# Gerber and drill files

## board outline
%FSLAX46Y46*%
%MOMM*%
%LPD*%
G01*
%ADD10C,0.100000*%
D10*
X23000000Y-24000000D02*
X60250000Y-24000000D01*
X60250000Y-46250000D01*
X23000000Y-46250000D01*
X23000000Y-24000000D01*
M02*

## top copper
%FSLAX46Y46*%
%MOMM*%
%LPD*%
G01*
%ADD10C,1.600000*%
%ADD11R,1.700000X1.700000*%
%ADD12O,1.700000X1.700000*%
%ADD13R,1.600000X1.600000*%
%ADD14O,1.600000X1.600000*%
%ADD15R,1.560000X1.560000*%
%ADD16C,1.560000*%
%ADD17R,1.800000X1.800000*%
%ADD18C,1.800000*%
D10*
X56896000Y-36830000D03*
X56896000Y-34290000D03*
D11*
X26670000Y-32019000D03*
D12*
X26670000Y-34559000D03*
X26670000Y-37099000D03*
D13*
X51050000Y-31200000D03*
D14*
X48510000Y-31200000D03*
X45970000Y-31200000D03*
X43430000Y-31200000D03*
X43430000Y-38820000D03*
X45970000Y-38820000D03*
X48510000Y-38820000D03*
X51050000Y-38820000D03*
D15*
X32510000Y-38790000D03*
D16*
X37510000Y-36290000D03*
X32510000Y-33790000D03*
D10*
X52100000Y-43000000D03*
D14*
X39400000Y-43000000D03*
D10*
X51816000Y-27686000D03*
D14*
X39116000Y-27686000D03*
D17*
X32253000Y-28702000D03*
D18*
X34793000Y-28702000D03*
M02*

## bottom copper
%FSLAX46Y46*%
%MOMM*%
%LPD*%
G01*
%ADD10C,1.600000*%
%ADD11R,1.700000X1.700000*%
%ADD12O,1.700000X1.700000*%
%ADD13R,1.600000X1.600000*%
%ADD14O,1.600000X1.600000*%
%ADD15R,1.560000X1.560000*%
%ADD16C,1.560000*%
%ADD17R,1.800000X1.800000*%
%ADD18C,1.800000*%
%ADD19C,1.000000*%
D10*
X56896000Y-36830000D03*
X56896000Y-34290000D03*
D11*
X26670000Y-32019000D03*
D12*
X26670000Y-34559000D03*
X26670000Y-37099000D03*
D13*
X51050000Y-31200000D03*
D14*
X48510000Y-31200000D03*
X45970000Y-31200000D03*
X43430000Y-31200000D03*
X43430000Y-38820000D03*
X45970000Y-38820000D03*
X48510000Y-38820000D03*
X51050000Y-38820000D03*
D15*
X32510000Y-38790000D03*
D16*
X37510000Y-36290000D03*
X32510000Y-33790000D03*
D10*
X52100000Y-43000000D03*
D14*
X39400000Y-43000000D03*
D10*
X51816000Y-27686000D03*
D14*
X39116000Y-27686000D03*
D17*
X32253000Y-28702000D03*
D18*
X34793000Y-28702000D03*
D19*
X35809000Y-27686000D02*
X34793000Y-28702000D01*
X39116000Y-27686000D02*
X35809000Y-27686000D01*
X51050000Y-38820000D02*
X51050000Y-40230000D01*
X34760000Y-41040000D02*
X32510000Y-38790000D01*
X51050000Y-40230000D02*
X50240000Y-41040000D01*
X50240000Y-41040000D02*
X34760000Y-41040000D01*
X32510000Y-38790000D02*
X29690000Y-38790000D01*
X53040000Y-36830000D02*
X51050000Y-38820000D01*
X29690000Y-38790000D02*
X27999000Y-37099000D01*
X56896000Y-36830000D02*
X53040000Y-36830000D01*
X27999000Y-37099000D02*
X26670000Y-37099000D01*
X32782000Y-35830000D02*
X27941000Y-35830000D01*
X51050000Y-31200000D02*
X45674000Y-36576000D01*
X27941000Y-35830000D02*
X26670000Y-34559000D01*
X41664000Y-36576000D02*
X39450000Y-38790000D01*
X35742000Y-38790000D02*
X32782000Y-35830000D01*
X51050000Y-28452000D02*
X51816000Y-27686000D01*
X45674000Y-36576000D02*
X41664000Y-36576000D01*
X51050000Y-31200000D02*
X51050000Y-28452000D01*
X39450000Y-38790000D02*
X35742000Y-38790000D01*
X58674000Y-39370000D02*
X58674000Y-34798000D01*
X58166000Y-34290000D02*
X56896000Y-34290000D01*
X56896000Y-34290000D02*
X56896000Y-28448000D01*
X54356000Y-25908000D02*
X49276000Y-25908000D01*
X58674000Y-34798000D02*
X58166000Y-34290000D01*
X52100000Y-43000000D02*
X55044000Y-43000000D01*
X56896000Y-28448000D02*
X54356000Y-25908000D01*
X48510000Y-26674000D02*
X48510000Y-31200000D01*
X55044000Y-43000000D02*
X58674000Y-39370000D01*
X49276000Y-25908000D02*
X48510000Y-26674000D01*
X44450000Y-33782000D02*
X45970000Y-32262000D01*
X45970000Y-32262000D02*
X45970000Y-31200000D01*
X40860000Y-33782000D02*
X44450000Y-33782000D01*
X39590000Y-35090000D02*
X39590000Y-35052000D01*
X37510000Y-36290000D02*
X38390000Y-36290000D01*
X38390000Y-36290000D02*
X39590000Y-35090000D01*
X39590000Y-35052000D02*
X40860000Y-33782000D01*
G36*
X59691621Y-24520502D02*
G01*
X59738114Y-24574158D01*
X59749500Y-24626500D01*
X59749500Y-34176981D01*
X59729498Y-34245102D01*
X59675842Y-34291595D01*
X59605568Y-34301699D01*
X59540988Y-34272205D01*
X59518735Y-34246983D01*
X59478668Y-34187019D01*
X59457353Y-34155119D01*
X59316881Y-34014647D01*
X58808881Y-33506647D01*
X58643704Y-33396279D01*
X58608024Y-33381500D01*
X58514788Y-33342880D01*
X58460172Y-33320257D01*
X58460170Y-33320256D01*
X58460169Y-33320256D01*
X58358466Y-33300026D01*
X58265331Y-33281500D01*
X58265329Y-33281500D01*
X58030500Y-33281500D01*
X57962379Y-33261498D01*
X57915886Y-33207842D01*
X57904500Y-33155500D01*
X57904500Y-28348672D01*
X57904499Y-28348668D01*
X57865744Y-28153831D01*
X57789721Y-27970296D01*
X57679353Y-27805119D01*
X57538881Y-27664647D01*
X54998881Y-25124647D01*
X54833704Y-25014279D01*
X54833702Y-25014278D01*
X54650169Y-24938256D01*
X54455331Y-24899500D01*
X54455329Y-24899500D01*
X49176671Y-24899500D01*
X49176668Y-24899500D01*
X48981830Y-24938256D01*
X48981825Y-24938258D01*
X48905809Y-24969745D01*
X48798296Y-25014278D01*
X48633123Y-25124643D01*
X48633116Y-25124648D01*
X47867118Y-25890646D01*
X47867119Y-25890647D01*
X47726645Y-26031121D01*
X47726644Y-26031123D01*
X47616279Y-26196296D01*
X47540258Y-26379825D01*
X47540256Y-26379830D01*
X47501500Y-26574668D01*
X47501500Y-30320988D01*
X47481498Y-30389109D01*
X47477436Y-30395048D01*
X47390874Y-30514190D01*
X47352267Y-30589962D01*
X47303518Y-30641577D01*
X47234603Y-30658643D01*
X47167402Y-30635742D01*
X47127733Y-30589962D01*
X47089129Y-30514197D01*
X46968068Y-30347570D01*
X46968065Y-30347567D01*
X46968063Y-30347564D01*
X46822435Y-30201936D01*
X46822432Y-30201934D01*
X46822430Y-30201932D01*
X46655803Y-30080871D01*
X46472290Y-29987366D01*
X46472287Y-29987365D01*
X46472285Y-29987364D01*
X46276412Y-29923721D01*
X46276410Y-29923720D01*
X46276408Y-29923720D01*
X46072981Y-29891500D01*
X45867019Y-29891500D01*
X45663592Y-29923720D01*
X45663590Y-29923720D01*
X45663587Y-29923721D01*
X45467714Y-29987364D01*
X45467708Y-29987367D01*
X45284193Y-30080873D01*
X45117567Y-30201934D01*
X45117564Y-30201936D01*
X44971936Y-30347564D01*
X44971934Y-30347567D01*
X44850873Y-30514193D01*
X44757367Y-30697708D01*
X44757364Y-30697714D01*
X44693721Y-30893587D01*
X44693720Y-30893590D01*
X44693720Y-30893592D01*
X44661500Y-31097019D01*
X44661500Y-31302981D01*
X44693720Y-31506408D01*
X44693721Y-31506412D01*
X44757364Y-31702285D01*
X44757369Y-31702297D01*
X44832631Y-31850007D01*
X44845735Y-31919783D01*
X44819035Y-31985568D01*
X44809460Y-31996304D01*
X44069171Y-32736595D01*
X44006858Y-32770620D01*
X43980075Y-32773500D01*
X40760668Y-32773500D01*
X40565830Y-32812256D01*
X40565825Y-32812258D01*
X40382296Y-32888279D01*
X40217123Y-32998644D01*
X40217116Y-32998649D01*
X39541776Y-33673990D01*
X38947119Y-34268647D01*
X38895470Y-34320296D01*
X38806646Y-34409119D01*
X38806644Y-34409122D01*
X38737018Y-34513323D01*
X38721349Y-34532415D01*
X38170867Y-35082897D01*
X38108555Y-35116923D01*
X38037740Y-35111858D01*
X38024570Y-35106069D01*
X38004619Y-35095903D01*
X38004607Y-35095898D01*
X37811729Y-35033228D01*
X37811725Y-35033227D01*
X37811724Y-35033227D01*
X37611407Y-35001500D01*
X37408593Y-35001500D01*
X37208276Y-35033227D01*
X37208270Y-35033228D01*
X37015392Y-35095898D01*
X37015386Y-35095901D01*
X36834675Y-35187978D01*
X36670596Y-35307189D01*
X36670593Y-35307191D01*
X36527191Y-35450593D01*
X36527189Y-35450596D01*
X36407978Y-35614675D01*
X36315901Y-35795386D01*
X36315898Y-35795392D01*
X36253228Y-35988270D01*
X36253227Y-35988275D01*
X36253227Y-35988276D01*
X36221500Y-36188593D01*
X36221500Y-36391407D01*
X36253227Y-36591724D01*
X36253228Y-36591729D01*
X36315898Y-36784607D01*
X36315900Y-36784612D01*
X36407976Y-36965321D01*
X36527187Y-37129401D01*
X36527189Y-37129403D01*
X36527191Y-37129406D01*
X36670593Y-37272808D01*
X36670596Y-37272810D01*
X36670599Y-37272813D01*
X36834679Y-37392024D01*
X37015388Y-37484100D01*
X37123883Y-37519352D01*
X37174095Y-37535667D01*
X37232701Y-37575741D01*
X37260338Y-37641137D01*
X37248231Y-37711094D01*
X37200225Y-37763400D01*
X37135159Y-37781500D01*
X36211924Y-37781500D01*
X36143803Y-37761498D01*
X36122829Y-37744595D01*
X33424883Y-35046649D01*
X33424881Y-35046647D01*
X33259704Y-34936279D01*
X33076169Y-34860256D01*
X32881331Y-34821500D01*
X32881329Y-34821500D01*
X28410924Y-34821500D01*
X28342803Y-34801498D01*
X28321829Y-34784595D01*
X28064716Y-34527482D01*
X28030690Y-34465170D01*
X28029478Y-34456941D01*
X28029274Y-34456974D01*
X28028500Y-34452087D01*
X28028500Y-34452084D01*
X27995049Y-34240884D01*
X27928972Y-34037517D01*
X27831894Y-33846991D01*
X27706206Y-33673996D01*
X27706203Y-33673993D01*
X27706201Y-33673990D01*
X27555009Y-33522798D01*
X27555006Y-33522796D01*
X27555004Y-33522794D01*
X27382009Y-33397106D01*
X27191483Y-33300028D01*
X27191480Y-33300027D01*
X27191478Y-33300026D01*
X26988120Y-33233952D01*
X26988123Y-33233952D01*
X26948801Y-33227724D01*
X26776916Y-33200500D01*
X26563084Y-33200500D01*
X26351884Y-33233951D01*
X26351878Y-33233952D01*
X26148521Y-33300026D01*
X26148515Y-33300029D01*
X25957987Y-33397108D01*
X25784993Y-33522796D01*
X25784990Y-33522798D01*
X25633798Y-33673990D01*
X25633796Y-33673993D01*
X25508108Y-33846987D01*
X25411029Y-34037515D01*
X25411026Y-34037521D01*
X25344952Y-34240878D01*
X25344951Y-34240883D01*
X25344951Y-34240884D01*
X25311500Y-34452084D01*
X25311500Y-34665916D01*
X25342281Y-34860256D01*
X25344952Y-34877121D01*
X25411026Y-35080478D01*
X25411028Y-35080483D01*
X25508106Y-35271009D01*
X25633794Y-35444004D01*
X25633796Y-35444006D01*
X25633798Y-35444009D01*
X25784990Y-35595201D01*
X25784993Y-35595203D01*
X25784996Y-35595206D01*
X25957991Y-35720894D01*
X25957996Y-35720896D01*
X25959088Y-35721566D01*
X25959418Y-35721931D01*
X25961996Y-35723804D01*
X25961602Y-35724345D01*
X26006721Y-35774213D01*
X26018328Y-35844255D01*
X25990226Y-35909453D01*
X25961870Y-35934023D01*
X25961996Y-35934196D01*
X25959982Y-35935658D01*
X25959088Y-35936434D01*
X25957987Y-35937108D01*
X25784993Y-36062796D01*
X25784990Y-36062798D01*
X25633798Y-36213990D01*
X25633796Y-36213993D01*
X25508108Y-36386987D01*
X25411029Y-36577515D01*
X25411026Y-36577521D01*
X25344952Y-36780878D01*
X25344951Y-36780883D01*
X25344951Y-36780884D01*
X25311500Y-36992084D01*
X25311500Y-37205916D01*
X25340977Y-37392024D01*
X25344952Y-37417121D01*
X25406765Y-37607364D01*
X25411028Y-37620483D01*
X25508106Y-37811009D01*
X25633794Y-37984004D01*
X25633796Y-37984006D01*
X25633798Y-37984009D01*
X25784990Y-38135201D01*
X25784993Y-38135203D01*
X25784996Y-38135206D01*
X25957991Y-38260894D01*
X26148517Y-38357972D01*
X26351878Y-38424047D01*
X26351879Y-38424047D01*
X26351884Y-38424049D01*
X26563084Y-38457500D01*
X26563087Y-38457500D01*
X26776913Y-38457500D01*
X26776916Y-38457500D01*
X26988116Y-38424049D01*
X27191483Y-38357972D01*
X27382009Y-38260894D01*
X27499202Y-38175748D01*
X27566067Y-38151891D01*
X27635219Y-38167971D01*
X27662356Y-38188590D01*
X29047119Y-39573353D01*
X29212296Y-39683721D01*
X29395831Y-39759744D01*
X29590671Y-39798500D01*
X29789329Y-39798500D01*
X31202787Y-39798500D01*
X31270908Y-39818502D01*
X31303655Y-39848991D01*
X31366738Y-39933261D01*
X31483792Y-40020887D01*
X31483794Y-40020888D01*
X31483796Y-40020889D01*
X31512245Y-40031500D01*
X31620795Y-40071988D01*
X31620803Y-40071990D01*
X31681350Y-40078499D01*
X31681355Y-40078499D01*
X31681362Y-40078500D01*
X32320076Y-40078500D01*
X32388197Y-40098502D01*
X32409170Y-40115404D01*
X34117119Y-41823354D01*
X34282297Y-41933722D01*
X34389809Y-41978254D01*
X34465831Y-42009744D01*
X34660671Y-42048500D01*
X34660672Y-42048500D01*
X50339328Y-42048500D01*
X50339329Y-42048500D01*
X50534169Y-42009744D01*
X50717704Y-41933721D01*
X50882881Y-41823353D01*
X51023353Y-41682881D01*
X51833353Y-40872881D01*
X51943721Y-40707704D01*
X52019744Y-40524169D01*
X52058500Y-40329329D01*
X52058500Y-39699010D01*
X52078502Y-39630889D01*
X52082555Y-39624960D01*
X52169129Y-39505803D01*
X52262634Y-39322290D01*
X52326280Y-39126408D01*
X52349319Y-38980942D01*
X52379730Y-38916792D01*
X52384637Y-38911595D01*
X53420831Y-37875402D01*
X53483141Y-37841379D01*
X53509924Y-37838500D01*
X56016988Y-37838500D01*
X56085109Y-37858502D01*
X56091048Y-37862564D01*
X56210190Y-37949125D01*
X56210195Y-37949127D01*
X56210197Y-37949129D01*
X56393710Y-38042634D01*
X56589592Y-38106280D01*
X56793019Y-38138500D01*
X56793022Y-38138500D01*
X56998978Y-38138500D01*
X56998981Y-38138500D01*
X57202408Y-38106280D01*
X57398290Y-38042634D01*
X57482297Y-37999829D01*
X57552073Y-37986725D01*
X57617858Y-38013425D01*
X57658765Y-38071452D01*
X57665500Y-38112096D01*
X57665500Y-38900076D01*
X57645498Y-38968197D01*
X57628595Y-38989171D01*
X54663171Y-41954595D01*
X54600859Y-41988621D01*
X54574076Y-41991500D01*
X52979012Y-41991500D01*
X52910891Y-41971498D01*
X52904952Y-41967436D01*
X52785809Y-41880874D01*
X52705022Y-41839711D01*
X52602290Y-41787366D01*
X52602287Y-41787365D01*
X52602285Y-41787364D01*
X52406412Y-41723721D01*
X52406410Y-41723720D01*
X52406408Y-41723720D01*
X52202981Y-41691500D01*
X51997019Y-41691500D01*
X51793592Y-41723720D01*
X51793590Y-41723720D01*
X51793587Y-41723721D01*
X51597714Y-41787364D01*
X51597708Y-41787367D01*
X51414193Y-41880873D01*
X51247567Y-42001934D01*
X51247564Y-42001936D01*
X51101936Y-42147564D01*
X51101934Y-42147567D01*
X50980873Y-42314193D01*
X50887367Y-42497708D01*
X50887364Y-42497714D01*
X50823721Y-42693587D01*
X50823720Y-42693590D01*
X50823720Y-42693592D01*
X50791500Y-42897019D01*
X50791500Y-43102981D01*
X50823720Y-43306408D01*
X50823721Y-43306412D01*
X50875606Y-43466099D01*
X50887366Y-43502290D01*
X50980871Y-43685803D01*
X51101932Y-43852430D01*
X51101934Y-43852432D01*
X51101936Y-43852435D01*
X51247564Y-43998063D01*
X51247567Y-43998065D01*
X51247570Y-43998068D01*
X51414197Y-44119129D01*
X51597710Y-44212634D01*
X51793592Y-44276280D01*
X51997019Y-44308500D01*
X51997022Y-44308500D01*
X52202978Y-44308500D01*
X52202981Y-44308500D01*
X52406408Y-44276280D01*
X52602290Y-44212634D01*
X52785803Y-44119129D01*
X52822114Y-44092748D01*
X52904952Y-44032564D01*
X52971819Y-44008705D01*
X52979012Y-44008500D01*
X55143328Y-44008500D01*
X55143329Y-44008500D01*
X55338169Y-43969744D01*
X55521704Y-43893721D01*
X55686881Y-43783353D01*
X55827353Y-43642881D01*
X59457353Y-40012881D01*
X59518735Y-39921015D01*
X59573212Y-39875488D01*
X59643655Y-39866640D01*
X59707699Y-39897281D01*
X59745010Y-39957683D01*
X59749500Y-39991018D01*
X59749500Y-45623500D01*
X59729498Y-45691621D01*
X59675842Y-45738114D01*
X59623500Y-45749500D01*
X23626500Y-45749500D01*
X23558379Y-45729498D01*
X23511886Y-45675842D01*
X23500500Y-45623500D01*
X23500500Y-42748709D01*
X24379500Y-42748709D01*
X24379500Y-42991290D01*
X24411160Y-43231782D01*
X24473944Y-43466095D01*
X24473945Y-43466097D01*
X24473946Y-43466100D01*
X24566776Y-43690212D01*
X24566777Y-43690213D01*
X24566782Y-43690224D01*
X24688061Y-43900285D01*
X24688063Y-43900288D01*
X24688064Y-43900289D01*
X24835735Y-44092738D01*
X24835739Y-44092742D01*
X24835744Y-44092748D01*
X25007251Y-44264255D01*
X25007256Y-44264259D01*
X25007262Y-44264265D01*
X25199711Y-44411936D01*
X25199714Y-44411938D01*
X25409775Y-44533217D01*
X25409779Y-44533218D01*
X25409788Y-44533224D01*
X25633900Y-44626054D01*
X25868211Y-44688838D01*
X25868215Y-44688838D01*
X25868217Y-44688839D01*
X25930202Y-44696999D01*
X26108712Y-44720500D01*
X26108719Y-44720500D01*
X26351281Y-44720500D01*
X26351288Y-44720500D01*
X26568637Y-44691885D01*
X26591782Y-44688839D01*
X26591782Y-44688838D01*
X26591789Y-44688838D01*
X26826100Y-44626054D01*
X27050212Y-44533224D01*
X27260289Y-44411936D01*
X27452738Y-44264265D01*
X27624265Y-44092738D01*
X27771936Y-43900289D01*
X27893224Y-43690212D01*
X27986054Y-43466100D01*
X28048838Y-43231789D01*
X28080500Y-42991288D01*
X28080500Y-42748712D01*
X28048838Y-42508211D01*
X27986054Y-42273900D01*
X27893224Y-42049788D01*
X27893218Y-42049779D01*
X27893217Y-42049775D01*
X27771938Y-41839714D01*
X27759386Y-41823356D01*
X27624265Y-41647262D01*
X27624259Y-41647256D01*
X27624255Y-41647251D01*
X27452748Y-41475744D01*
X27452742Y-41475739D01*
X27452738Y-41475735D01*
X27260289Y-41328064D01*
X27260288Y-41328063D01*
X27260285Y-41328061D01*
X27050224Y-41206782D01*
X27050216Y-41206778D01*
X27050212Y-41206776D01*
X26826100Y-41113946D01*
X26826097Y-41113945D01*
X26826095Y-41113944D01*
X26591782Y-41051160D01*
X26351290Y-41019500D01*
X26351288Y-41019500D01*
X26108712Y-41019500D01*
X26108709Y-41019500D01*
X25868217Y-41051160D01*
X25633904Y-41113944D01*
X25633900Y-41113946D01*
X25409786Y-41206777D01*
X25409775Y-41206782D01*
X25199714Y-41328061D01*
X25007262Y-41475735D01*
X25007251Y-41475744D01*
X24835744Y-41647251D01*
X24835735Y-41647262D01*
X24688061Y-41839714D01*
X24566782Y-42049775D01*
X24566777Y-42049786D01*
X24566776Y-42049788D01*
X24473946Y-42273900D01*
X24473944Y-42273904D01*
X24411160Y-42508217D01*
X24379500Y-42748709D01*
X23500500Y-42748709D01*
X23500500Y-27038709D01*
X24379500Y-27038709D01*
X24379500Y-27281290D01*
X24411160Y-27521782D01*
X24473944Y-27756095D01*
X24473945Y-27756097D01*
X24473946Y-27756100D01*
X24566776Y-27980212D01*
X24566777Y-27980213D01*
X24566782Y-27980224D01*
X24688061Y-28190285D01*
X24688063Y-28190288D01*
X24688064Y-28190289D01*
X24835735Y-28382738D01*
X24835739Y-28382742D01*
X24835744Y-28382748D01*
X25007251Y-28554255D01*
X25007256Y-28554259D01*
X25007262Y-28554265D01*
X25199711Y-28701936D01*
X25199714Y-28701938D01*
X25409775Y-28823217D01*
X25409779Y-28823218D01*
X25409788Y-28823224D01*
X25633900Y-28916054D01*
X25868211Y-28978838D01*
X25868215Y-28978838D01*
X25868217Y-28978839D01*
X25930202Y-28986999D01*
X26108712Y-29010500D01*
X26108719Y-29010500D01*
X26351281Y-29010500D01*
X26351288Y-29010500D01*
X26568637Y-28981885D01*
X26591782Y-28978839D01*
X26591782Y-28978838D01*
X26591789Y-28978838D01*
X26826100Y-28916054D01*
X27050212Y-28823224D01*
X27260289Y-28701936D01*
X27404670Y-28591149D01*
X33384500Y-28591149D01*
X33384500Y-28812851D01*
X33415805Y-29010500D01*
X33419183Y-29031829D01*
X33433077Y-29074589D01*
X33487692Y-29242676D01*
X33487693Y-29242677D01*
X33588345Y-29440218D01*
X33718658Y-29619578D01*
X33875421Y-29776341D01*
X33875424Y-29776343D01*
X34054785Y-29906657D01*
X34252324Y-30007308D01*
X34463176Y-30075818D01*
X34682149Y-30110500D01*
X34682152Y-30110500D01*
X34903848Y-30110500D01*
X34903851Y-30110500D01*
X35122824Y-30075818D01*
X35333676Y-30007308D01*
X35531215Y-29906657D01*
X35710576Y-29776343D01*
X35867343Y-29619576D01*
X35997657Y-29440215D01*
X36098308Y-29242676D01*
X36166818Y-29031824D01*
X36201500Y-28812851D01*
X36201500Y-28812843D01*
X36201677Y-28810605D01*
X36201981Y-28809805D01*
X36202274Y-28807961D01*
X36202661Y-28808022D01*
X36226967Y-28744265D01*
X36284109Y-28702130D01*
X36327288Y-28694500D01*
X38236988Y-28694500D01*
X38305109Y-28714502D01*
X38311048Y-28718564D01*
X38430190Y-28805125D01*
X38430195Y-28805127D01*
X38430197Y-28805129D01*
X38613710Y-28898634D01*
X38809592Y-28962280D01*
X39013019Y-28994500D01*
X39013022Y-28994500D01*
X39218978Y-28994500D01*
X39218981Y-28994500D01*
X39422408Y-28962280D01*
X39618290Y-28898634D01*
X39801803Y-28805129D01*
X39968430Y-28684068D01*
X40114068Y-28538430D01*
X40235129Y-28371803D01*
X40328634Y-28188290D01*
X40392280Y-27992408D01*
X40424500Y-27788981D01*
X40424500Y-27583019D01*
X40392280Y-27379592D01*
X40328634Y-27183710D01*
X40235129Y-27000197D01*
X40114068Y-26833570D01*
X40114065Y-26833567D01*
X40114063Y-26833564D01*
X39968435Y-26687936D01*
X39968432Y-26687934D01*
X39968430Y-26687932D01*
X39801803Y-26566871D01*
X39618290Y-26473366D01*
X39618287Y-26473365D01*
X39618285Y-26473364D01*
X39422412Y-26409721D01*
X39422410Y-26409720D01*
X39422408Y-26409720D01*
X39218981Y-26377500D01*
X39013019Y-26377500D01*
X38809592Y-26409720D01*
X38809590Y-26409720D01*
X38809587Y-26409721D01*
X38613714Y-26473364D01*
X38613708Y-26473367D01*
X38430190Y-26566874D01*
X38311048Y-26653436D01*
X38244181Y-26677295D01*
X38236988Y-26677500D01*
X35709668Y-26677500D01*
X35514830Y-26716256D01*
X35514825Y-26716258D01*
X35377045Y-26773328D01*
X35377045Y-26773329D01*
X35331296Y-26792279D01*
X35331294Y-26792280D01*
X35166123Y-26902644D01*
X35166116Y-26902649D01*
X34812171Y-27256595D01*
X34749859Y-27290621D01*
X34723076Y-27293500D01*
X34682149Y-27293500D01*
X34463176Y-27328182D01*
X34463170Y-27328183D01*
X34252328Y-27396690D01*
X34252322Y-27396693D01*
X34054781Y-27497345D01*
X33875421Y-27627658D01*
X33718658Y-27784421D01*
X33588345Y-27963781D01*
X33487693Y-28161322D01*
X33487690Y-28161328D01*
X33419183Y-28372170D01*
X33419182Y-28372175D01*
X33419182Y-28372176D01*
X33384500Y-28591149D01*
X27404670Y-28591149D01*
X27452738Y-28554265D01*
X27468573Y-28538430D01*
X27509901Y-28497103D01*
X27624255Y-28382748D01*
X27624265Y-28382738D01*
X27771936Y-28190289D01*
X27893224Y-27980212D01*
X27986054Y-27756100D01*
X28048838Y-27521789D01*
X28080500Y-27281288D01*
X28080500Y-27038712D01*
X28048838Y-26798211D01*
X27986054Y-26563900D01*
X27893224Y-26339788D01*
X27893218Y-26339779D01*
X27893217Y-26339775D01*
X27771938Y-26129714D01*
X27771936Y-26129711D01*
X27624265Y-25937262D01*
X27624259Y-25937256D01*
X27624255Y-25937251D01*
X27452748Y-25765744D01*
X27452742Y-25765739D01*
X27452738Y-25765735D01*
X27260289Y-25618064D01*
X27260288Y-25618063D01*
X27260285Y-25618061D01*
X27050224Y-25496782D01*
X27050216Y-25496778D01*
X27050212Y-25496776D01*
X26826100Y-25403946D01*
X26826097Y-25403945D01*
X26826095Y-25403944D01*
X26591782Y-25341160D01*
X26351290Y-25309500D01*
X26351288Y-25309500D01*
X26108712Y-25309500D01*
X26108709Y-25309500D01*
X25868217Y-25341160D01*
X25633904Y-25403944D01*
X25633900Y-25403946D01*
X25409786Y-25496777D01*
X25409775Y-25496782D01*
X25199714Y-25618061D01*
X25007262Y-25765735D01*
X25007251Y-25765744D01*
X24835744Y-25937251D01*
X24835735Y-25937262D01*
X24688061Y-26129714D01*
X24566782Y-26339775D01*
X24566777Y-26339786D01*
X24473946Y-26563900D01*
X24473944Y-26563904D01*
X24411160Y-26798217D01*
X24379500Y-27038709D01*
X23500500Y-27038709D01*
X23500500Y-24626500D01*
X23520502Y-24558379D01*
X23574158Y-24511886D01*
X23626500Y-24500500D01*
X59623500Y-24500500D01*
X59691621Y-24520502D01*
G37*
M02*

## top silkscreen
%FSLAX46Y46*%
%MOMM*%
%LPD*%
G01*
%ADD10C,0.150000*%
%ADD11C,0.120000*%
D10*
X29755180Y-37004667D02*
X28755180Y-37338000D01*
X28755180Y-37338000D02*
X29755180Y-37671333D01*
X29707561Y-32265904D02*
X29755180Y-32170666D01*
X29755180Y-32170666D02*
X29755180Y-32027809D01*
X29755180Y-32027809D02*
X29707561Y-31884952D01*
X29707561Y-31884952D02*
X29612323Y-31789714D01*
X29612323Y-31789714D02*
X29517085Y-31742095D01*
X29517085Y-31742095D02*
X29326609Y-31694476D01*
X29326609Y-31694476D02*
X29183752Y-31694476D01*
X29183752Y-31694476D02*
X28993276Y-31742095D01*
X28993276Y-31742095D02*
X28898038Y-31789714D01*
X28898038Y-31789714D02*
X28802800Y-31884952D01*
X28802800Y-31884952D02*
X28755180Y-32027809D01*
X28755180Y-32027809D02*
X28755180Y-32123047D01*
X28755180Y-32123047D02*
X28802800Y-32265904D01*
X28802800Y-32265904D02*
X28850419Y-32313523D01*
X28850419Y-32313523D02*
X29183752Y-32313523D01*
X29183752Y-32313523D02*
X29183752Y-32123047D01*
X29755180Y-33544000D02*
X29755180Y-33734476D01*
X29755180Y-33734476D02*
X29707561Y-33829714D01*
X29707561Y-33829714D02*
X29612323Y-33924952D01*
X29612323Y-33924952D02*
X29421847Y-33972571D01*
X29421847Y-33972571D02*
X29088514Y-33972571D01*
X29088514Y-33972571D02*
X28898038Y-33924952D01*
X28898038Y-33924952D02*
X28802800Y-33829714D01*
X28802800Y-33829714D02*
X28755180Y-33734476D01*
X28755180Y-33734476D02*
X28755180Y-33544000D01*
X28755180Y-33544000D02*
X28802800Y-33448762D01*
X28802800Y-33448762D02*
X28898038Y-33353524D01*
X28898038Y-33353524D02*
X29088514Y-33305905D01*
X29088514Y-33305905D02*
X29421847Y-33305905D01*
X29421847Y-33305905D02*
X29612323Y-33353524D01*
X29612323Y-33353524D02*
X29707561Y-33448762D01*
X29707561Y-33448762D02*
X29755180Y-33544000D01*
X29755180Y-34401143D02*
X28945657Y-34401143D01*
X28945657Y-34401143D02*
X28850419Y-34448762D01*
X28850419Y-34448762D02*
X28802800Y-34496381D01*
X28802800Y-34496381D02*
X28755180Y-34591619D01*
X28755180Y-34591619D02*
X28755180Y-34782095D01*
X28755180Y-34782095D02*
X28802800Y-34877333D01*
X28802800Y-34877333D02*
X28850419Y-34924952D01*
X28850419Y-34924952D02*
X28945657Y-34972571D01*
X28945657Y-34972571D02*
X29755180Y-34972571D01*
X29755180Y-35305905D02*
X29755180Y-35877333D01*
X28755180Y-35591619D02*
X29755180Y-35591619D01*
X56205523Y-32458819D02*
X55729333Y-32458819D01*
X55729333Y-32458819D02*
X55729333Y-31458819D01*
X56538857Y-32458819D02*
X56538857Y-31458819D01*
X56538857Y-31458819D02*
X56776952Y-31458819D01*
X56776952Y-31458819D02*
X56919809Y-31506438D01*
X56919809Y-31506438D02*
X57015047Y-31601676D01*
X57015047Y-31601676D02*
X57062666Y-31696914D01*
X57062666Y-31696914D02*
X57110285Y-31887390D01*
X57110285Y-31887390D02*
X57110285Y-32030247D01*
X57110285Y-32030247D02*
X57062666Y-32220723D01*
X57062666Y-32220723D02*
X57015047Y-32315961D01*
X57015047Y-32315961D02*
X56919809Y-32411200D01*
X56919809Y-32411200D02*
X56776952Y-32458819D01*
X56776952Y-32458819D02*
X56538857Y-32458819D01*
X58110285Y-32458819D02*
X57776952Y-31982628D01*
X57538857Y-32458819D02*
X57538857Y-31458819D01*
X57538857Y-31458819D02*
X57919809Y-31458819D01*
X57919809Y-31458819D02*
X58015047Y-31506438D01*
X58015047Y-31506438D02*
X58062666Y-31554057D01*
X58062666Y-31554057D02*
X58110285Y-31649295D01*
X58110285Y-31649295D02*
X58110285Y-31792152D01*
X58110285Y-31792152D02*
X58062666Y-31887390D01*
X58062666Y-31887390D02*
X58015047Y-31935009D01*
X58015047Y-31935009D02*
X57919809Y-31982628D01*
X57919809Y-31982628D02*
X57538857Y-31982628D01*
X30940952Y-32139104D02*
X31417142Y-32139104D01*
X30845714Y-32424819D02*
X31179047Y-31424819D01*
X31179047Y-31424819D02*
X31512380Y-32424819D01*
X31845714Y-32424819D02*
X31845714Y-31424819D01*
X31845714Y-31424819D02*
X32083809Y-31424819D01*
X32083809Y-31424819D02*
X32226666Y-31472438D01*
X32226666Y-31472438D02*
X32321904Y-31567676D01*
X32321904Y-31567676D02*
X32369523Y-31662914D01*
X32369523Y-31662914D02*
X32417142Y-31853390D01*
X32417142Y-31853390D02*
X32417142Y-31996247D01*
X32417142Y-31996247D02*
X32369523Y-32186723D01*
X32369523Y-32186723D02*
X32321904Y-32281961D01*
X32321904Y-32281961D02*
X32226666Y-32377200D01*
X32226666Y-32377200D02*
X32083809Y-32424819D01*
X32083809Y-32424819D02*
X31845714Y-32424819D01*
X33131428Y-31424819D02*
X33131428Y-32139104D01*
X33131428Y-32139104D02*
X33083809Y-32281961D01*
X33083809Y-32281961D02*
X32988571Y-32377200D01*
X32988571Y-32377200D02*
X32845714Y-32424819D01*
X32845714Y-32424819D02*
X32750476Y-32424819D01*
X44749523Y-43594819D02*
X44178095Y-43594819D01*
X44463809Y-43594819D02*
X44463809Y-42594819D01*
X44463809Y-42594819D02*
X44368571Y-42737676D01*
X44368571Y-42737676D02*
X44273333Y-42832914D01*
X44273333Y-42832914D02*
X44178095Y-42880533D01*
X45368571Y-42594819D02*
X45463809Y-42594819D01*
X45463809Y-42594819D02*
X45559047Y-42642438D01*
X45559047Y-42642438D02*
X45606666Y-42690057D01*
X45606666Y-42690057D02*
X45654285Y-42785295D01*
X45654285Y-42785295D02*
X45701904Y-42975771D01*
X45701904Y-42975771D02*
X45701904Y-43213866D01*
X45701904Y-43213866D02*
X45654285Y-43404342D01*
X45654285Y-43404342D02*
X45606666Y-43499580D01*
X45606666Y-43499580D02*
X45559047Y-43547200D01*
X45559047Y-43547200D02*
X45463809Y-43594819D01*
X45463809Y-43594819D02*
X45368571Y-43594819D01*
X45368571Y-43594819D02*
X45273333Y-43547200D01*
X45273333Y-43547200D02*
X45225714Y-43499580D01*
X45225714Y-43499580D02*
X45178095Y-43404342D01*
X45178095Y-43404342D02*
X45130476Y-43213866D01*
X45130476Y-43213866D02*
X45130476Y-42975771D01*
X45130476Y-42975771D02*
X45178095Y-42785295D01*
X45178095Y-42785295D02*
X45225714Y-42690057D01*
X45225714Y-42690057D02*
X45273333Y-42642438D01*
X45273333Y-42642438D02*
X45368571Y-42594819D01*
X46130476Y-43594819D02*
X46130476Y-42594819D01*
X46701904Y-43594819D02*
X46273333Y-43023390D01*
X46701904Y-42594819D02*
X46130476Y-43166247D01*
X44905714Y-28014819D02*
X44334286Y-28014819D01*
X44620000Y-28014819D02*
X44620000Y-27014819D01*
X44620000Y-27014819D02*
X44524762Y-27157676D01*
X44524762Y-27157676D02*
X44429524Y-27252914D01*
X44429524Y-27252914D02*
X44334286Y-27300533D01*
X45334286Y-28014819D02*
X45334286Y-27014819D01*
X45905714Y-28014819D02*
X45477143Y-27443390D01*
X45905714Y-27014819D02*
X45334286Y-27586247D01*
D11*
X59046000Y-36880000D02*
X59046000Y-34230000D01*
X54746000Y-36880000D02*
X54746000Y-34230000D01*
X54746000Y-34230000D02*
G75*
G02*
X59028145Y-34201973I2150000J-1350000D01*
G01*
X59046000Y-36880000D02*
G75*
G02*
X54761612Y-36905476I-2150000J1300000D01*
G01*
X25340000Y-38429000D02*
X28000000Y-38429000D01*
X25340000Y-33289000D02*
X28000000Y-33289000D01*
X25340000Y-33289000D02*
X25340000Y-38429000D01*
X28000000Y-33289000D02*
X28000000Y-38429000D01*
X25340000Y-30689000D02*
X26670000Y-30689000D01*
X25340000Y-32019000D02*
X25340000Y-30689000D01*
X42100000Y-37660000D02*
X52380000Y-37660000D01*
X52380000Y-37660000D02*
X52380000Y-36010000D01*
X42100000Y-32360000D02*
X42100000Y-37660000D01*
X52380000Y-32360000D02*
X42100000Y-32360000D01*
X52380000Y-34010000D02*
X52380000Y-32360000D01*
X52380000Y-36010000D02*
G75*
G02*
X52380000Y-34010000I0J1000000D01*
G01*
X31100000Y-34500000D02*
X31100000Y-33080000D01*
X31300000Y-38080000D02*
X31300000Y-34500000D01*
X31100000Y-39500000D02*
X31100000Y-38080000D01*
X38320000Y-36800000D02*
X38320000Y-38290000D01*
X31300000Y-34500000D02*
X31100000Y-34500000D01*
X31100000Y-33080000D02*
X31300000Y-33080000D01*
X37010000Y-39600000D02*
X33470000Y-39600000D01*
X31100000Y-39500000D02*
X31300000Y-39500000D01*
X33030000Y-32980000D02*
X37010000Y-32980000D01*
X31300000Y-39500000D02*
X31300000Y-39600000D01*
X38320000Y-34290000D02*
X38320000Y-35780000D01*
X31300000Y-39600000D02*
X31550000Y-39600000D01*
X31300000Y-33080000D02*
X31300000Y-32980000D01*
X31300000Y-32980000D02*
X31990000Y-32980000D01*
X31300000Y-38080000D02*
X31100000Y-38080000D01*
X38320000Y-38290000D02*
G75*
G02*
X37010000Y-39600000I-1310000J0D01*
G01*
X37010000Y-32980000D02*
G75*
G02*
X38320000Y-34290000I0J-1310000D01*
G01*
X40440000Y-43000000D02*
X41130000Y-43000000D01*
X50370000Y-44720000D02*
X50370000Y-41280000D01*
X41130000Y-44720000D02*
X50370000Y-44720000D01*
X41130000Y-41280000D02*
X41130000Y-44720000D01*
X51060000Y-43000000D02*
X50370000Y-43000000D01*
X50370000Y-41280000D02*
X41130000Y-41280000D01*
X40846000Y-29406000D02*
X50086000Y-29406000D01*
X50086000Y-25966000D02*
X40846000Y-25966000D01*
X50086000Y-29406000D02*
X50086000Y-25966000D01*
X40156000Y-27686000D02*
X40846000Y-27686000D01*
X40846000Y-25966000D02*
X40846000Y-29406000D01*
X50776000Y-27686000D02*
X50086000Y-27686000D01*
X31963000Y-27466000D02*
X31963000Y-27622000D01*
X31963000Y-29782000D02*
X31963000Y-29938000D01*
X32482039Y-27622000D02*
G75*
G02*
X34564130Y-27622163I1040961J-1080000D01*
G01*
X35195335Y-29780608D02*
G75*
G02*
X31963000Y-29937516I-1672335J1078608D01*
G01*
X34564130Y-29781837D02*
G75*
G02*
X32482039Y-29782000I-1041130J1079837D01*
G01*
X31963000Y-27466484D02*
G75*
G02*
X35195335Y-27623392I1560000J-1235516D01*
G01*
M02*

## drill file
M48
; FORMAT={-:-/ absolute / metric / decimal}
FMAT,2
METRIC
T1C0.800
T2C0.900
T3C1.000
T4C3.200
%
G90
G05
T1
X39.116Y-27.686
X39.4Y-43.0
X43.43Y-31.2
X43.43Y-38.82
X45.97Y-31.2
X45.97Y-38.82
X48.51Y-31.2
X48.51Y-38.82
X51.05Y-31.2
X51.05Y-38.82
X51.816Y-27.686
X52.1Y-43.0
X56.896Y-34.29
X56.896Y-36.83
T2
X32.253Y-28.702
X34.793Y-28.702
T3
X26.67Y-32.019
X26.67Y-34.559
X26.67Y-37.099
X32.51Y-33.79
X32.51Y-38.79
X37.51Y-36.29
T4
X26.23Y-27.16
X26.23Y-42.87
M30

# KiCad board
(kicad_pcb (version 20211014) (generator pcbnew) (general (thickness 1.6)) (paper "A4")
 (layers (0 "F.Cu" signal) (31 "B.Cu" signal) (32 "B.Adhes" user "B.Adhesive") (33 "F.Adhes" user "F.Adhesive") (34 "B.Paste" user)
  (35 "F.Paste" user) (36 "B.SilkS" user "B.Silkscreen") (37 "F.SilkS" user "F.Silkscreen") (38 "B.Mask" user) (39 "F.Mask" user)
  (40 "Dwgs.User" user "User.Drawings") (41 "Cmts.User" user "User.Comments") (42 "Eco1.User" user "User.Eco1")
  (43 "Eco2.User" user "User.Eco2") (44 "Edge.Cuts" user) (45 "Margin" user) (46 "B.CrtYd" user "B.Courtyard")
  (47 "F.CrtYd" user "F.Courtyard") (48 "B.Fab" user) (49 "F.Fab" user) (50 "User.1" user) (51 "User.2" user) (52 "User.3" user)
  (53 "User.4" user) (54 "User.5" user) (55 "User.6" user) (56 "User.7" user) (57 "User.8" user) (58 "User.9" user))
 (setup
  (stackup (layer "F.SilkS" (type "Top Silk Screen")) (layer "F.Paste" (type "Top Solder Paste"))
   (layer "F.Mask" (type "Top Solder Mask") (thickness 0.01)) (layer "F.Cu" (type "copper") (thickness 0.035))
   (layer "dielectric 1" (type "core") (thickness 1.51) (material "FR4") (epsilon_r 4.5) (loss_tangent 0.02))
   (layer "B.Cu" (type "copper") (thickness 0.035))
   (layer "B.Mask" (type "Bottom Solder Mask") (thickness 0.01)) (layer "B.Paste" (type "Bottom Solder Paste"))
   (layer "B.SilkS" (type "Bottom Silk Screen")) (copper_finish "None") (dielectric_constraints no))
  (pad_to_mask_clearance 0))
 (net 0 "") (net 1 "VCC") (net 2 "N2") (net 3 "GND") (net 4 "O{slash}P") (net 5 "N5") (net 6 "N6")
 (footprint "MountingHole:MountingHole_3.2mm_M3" (layer "F.Cu") (at 26.23 27.16)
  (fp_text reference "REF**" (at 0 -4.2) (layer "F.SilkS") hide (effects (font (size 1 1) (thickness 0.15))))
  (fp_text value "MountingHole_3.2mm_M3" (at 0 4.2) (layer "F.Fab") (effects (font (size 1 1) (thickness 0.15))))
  (pad "" np_thru_hole circle (at 0 0) (size 3.2 3.2) (drill 3.2) (layers *.Cu *.Mask)))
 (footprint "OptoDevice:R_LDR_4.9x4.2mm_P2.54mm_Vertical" (layer "F.Cu") (at 56.896 36.83 90)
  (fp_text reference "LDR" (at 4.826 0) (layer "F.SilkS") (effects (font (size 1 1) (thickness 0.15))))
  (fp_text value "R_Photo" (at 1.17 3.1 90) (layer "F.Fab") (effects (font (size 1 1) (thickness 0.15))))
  (fp_line (start -0.05 2.15) (end 2.6 2.15) (layer "F.SilkS") (width 0.12))
  (fp_line (start -0.05 -2.15) (end 2.6 -2.15) (layer "F.SilkS") (width 0.12))
  (fp_arc (start 2.6 -2.15) (mid 3.788646 -0.016616) (end 2.628027 2.132145) (layer "F.SilkS") (width 0.12))
  (fp_arc (start -0.05 2.15) (mid -1.262424 0.01494) (end -0.075476 -2.134388) (layer "F.SilkS") (width 0.12))
  (pad "1" thru_hole circle (at 0 0 90) (size 1.6 1.6) (drill 0.8) (layers *.Cu *.Mask) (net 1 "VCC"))
  (pad "2" thru_hole circle (at 2.54 0 90) (size 1.6 1.6) (drill 0.8) (layers *.Cu *.Mask) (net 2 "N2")))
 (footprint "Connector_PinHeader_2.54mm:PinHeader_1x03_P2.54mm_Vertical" (layer "F.Cu") (at 26.67 32.019)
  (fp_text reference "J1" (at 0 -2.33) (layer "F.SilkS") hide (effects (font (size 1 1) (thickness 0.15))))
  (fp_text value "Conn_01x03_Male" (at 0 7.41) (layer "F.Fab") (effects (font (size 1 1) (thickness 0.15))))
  (fp_line (start -1.33 6.41) (end 1.33 6.41) (layer "F.SilkS") (width 0.12))
  (fp_line (start -1.33 1.27) (end 1.33 1.27) (layer "F.SilkS") (width 0.12))
  (fp_line (start -1.33 1.27) (end -1.33 6.41) (layer "F.SilkS") (width 0.12))
  (fp_line (start 1.33 1.27) (end 1.33 6.41) (layer "F.SilkS") (width 0.12))
  (fp_line (start -1.33 -1.33) (end 0 -1.33) (layer "F.SilkS") (width 0.12))
  (fp_line (start -1.33 0) (end -1.33 -1.33) (layer "F.SilkS") (width 0.12))
  (pad "1" thru_hole rect (at 0 0) (size 1.7 1.7) (drill 1) (layers *.Cu *.Mask) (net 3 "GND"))
  (pad "2" thru_hole oval (at 0 2.54) (size 1.7 1.7) (drill 1) (layers *.Cu *.Mask) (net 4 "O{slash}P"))
  (pad "3" thru_hole oval (at 0 5.08) (size 1.7 1.7) (drill 1) (layers *.Cu *.Mask) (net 1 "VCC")))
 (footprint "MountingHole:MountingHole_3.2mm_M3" (layer "F.Cu") (at 26.23 42.87)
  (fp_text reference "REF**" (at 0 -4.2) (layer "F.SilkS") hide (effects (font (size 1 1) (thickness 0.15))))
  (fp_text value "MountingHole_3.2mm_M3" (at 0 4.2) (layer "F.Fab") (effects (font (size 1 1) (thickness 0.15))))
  (pad "" np_thru_hole circle (at 0 0) (size 3.2 3.2) (drill 3.2) (layers *.Cu *.Mask)))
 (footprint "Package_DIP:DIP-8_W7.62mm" (layer "F.Cu") (at 51.05 31.2 -90)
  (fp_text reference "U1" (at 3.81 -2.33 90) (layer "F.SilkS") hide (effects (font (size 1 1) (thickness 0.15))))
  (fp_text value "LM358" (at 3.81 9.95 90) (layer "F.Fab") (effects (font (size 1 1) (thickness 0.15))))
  (fp_line (start 6.46 8.95) (end 6.46 -1.33) (layer "F.SilkS") (width 0.12))
  (fp_line (start 6.46 -1.33) (end 4.81 -1.33) (layer "F.SilkS") (width 0.12))
  (fp_line (start 1.16 8.95) (end 6.46 8.95) (layer "F.SilkS") (width 0.12))
  (fp_line (start 1.16 -1.33) (end 1.16 8.95) (layer "F.SilkS") (width 0.12))
  (fp_line (start 2.81 -1.33) (end 1.16 -1.33) (layer "F.SilkS") (width 0.12))
  (fp_arc (start 4.81 -1.33) (mid 3.81 -0.33) (end 2.81 -1.33) (layer "F.SilkS") (width 0.12))
  (pad "1" thru_hole rect (at 0 0 270) (size 1.6 1.6) (drill 0.8) (layers *.Cu *.Mask) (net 4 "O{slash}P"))
  (pad "2" thru_hole oval (at 0 2.54 270) (size 1.6 1.6) (drill 0.8) (layers *.Cu *.Mask) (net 2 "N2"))
  (pad "3" thru_hole oval (at 0 5.08 270) (size 1.6 1.6) (drill 0.8) (layers *.Cu *.Mask) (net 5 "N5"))
  (pad "4" thru_hole oval (at 0 7.62 270) (size 1.6 1.6) (drill 0.8) (layers *.Cu *.Mask) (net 3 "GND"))
  (pad "5" thru_hole oval (at 7.62 7.62 270) (size 1.6 1.6) (drill 0.8) (layers *.Cu *.Mask))
  (pad "6" thru_hole oval (at 7.62 5.08 270) (size 1.6 1.6) (drill 0.8) (layers *.Cu *.Mask))
  (pad "7" thru_hole oval (at 7.62 2.54 270) (size 1.6 1.6) (drill 0.8) (layers *.Cu *.Mask))
  (pad "8" thru_hole oval (at 7.62 0 270) (size 1.6 1.6) (drill 0.8) (layers *.Cu *.Mask) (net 1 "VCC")))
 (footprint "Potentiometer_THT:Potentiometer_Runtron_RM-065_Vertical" (layer "F.Cu") (at 32.51 38.79 90)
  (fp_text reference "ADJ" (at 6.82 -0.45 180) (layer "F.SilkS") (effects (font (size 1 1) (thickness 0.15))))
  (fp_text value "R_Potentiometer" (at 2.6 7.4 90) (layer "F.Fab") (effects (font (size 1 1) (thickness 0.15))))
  (fp_line (start 4.29 -1.41) (end 5.71 -1.41) (layer "F.SilkS") (width 0.12))
  (fp_line (start 0.71 -1.21) (end 4.29 -1.21) (layer "F.SilkS") (width 0.12))
  (fp_line (start -0.71 -1.41) (end 0.71 -1.41) (layer "F.SilkS") (width 0.12))
  (fp_line (start 1.99 5.81) (end 0.5 5.81) (layer "F.SilkS") (width 0.12))
  (fp_line (start 4.29 -1.21) (end 4.29 -1.41) (layer "F.SilkS") (width 0.12))
  (fp_line (start 5.71 -1.41) (end 5.71 -1.21) (layer "F.SilkS") (width 0.12))
  (fp_line (start -0.81 4.5) (end -0.81 0.96) (layer "F.SilkS") (width 0.12))
  (fp_line (start -0.71 -1.41) (end -0.71 -1.21) (layer "F.SilkS") (width 0.12))
  (fp_line (start 5.81 0.52) (end 5.81 4.5) (layer "F.SilkS") (width 0.12))
  (fp_line (start -0.71 -1.21) (end -0.81 -1.21) (layer "F.SilkS") (width 0.12))
  (fp_line (start 4.5 5.81) (end 3.01 5.81) (layer "F.SilkS") (width 0.12))
  (fp_line (start -0.81 -1.21) (end -0.81 -0.96) (layer "F.SilkS") (width 0.12))
  (fp_line (start 5.71 -1.21) (end 5.81 -1.21) (layer "F.SilkS") (width 0.12))
  (fp_line (start 5.81 -1.21) (end 5.81 -0.52) (layer "F.SilkS") (width 0.12))
  (fp_line (start 0.71 -1.21) (end 0.71 -1.41) (layer "F.SilkS") (width 0.12))
  (fp_arc (start 0.5 5.81) (mid -0.42631 5.42631) (end -0.81 4.5) (layer "F.SilkS") (width 0.12))
  (fp_arc (start 5.81 4.5) (mid 5.42631 5.42631) (end 4.5 5.81) (layer "F.SilkS") (width 0.12))
  (pad "1" thru_hole rect (at 0 0 90) (size 1.56 1.56) (drill 1) (layers *.Cu *.Mask) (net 1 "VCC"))
  (pad "2" thru_hole circle (at 2.5 5 90) (size 1.56 1.56) (drill 1) (layers *.Cu *.Mask) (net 5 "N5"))
  (pad "3" thru_hole circle (at 5 0 90) (size 1.56 1.56) (drill 1) (layers *.Cu *.Mask) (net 3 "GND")))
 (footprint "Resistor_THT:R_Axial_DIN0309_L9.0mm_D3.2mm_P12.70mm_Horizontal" (layer "F.Cu") (at 52.1 43 180)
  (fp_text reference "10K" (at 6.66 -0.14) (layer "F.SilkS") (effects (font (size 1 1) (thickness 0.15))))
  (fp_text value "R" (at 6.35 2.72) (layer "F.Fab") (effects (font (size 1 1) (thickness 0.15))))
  (fp_line (start 11.66 0) (end 10.97 0) (layer "F.SilkS") (width 0.12))
  (fp_line (start 1.73 -1.72) (end 1.73 1.72) (layer "F.SilkS") (width 0.12))
  (fp_line (start 10.97 -1.72) (end 1.73 -1.72) (layer "F.SilkS") (width 0.12))
  (fp_line (start 10.97 1.72) (end 10.97 -1.72) (layer "F.SilkS") (width 0.12))
  (fp_line (start 1.04 0) (end 1.73 0) (layer "F.SilkS") (width 0.12))
  (fp_line (start 1.73 1.72) (end 10.97 1.72) (layer "F.SilkS") (width 0.12))
  (pad "1" thru_hole circle (at 0 0 180) (size 1.6 1.6) (drill 0.8) (layers *.Cu *.Mask) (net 2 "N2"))
  (pad "2" thru_hole oval (at 12.7 0 180) (size 1.6 1.6) (drill 0.8) (layers *.Cu *.Mask) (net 3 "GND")))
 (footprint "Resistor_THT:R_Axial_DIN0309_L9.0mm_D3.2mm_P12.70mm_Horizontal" (layer "F.Cu") (at 51.816 27.686 180)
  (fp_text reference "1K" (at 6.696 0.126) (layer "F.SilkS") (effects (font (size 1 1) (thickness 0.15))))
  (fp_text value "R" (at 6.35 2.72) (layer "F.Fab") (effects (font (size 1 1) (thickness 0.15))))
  (fp_line (start 10.97 -1.72) (end 1.73 -1.72) (layer "F.SilkS") (width 0.12))
  (fp_line (start 1.73 1.72) (end 10.97 1.72) (layer "F.SilkS") (width 0.12))
  (fp_line (start 1.73 -1.72) (end 1.73 1.72) (layer "F.SilkS") (width 0.12))
  (fp_line (start 11.66 0) (end 10.97 0) (layer "F.SilkS") (width 0.12))
  (fp_line (start 10.97 1.72) (end 10.97 -1.72) (layer "F.SilkS") (width 0.12))
  (fp_line (start 1.04 0) (end 1.73 0) (layer "F.SilkS") (width 0.12))
  (pad "1" thru_hole circle (at 0 0 180) (size 1.6 1.6) (drill 0.8) (layers *.Cu *.Mask) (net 4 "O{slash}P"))
  (pad "2" thru_hole oval (at 12.7 0 180) (size 1.6 1.6) (drill 0.8) (layers *.Cu *.Mask) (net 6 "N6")))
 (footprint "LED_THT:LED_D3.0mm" (layer "F.Cu") (at 32.253 28.702)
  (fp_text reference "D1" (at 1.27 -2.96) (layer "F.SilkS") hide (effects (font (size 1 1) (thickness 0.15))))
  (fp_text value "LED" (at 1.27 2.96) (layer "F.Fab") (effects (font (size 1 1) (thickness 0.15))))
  (fp_line (start -0.29 -1.236) (end -0.29 -1.08) (layer "F.SilkS") (width 0.12))
  (fp_line (start -0.29 1.08) (end -0.29 1.236) (layer "F.SilkS") (width 0.12))
  (fp_arc (start 0.229039 -1.08) (mid 1.270117 -1.5) (end 2.31113 -1.079837) (layer "F.SilkS") (width 0.12))
  (fp_arc (start 2.942335 1.078608) (mid 1.366487 1.987659) (end -0.29 1.235516) (layer "F.SilkS") (width 0.12))
  (fp_arc (start 2.31113 1.079837) (mid 1.270117 1.5) (end 0.229039 1.08) (layer "F.SilkS") (width 0.12))
  (fp_arc (start -0.29 -1.235516) (mid 1.366487 -1.987659) (end 2.942335 -1.078608) (layer "F.SilkS") (width 0.12))
  (pad "1" thru_hole rect (at 0 0) (size 1.8 1.8) (drill 0.9) (layers *.Cu *.Mask) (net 3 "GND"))
  (pad "2" thru_hole circle (at 2.54 0) (size 1.8 1.8) (drill 0.9) (layers *.Cu *.Mask) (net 6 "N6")))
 (gr_rect (start 23 24) (end 60.25 46.25) (layer "Edge.Cuts") (width 0.1) (fill none))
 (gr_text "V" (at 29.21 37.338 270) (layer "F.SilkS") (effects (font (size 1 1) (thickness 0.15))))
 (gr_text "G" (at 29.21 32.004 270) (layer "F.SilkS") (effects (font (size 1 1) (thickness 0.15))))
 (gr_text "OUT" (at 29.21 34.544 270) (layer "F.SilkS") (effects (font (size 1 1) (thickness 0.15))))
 (segment (start 35.809 27.686) (end 34.793 28.702) (width 1) (layer "B.Cu") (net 6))
 (segment (start 39.116 27.686) (end 35.809 27.686) (width 1) (layer "B.Cu") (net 6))
 (segment (start 51.05 38.82) (end 51.05 40.23) (width 1) (layer "B.Cu") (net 1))
 (segment (start 34.76 41.04) (end 32.51 38.79) (width 1) (layer "B.Cu") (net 1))
 (segment (start 51.05 40.23) (end 50.24 41.04) (width 1) (layer "B.Cu") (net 1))
 (segment (start 50.24 41.04) (end 34.76 41.04) (width 1) (layer "B.Cu") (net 1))
 (segment (start 32.51 38.79) (end 29.69 38.79) (width 1) (layer "B.Cu") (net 1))
 (segment (start 53.04 36.83) (end 51.05 38.82) (width 1) (layer "B.Cu") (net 1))
 (segment (start 29.69 38.79) (end 27.999 37.099) (width 1) (layer "B.Cu") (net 1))
 (segment (start 56.896 36.83) (end 53.04 36.83) (width 1) (layer "B.Cu") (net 1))
 (segment (start 27.999 37.099) (end 26.67 37.099) (width 1) (layer "B.Cu") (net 1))
 (segment (start 32.782 35.83) (end 27.941 35.83) (width 1) (layer "B.Cu") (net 4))
 (segment (start 51.05 31.2) (end 45.674 36.576) (width 1) (layer "B.Cu") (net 4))
 (segment (start 27.941 35.83) (end 26.67 34.559) (width 1) (layer "B.Cu") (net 4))
 (segment (start 41.664 36.576) (end 39.45 38.79) (width 1) (layer "B.Cu") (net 4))
 (segment (start 35.742 38.79) (end 32.782 35.83) (width 1) (layer "B.Cu") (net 4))
 (segment (start 51.05 28.452) (end 51.816 27.686) (width 1) (layer "B.Cu") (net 4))
 (segment (start 45.674 36.576) (end 41.664 36.576) (width 1) (layer "B.Cu") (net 4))
 (segment (start 51.05 31.2) (end 51.05 28.452) (width 1) (layer "B.Cu") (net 4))
 (segment (start 39.45 38.79) (end 35.742 38.79) (width 1) (layer "B.Cu") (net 4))
 (segment (start 58.674 39.37) (end 58.674 34.798) (width 1) (layer "B.Cu") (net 2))
 (segment (start 58.166 34.29) (end 56.896 34.29) (width 1) (layer "B.Cu") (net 2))
 (segment (start 56.896 34.29) (end 56.896 28.448) (width 1) (layer "B.Cu") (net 2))
 (segment (start 54.356 25.908) (end 49.276 25.908) (width 1) (layer "B.Cu") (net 2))
 (segment (start 58.674 34.798) (end 58.166 34.29) (width 1) (layer "B.Cu") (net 2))
 (segment (start 52.1 43) (end 55.044 43) (width 1) (layer "B.Cu") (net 2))
 (segment (start 56.896 28.448) (end 54.356 25.908) (width 1) (layer "B.Cu") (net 2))
 (segment (start 48.51 26.674) (end 48.51 31.2) (width 1) (layer "B.Cu") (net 2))
 (segment (start 55.044 43) (end 58.674 39.37) (width 1) (layer "B.Cu") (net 2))
 (segment (start 49.276 25.908) (end 48.51 26.674) (width 1) (layer "B.Cu") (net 2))
 (segment (start 44.45 33.782) (end 45.97 32.262) (width 1) (layer "B.Cu") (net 5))
 (segment (start 45.97 32.262) (end 45.97 31.2) (width 1) (layer "B.Cu") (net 5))
 (segment (start 40.86 33.782) (end 44.45 33.782) (width 1) (layer "B.Cu") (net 5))
 (segment (start 39.59 35.09) (end 39.59 35.052) (width 1) (layer "B.Cu") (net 5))
 (segment (start 37.51 36.29) (end 38.39 36.29) (width 1) (layer "B.Cu") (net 5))
 (segment (start 38.39 36.29) (end 39.59 35.09) (width 1) (layer "B.Cu") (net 5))
 (segment (start 39.59 35.052) (end 40.86 33.782) (width 1) (layer "B.Cu") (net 5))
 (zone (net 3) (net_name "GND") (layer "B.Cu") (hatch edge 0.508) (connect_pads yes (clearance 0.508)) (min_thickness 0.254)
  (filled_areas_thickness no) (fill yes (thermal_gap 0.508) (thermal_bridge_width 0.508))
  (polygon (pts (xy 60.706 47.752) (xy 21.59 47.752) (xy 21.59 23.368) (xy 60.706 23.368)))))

